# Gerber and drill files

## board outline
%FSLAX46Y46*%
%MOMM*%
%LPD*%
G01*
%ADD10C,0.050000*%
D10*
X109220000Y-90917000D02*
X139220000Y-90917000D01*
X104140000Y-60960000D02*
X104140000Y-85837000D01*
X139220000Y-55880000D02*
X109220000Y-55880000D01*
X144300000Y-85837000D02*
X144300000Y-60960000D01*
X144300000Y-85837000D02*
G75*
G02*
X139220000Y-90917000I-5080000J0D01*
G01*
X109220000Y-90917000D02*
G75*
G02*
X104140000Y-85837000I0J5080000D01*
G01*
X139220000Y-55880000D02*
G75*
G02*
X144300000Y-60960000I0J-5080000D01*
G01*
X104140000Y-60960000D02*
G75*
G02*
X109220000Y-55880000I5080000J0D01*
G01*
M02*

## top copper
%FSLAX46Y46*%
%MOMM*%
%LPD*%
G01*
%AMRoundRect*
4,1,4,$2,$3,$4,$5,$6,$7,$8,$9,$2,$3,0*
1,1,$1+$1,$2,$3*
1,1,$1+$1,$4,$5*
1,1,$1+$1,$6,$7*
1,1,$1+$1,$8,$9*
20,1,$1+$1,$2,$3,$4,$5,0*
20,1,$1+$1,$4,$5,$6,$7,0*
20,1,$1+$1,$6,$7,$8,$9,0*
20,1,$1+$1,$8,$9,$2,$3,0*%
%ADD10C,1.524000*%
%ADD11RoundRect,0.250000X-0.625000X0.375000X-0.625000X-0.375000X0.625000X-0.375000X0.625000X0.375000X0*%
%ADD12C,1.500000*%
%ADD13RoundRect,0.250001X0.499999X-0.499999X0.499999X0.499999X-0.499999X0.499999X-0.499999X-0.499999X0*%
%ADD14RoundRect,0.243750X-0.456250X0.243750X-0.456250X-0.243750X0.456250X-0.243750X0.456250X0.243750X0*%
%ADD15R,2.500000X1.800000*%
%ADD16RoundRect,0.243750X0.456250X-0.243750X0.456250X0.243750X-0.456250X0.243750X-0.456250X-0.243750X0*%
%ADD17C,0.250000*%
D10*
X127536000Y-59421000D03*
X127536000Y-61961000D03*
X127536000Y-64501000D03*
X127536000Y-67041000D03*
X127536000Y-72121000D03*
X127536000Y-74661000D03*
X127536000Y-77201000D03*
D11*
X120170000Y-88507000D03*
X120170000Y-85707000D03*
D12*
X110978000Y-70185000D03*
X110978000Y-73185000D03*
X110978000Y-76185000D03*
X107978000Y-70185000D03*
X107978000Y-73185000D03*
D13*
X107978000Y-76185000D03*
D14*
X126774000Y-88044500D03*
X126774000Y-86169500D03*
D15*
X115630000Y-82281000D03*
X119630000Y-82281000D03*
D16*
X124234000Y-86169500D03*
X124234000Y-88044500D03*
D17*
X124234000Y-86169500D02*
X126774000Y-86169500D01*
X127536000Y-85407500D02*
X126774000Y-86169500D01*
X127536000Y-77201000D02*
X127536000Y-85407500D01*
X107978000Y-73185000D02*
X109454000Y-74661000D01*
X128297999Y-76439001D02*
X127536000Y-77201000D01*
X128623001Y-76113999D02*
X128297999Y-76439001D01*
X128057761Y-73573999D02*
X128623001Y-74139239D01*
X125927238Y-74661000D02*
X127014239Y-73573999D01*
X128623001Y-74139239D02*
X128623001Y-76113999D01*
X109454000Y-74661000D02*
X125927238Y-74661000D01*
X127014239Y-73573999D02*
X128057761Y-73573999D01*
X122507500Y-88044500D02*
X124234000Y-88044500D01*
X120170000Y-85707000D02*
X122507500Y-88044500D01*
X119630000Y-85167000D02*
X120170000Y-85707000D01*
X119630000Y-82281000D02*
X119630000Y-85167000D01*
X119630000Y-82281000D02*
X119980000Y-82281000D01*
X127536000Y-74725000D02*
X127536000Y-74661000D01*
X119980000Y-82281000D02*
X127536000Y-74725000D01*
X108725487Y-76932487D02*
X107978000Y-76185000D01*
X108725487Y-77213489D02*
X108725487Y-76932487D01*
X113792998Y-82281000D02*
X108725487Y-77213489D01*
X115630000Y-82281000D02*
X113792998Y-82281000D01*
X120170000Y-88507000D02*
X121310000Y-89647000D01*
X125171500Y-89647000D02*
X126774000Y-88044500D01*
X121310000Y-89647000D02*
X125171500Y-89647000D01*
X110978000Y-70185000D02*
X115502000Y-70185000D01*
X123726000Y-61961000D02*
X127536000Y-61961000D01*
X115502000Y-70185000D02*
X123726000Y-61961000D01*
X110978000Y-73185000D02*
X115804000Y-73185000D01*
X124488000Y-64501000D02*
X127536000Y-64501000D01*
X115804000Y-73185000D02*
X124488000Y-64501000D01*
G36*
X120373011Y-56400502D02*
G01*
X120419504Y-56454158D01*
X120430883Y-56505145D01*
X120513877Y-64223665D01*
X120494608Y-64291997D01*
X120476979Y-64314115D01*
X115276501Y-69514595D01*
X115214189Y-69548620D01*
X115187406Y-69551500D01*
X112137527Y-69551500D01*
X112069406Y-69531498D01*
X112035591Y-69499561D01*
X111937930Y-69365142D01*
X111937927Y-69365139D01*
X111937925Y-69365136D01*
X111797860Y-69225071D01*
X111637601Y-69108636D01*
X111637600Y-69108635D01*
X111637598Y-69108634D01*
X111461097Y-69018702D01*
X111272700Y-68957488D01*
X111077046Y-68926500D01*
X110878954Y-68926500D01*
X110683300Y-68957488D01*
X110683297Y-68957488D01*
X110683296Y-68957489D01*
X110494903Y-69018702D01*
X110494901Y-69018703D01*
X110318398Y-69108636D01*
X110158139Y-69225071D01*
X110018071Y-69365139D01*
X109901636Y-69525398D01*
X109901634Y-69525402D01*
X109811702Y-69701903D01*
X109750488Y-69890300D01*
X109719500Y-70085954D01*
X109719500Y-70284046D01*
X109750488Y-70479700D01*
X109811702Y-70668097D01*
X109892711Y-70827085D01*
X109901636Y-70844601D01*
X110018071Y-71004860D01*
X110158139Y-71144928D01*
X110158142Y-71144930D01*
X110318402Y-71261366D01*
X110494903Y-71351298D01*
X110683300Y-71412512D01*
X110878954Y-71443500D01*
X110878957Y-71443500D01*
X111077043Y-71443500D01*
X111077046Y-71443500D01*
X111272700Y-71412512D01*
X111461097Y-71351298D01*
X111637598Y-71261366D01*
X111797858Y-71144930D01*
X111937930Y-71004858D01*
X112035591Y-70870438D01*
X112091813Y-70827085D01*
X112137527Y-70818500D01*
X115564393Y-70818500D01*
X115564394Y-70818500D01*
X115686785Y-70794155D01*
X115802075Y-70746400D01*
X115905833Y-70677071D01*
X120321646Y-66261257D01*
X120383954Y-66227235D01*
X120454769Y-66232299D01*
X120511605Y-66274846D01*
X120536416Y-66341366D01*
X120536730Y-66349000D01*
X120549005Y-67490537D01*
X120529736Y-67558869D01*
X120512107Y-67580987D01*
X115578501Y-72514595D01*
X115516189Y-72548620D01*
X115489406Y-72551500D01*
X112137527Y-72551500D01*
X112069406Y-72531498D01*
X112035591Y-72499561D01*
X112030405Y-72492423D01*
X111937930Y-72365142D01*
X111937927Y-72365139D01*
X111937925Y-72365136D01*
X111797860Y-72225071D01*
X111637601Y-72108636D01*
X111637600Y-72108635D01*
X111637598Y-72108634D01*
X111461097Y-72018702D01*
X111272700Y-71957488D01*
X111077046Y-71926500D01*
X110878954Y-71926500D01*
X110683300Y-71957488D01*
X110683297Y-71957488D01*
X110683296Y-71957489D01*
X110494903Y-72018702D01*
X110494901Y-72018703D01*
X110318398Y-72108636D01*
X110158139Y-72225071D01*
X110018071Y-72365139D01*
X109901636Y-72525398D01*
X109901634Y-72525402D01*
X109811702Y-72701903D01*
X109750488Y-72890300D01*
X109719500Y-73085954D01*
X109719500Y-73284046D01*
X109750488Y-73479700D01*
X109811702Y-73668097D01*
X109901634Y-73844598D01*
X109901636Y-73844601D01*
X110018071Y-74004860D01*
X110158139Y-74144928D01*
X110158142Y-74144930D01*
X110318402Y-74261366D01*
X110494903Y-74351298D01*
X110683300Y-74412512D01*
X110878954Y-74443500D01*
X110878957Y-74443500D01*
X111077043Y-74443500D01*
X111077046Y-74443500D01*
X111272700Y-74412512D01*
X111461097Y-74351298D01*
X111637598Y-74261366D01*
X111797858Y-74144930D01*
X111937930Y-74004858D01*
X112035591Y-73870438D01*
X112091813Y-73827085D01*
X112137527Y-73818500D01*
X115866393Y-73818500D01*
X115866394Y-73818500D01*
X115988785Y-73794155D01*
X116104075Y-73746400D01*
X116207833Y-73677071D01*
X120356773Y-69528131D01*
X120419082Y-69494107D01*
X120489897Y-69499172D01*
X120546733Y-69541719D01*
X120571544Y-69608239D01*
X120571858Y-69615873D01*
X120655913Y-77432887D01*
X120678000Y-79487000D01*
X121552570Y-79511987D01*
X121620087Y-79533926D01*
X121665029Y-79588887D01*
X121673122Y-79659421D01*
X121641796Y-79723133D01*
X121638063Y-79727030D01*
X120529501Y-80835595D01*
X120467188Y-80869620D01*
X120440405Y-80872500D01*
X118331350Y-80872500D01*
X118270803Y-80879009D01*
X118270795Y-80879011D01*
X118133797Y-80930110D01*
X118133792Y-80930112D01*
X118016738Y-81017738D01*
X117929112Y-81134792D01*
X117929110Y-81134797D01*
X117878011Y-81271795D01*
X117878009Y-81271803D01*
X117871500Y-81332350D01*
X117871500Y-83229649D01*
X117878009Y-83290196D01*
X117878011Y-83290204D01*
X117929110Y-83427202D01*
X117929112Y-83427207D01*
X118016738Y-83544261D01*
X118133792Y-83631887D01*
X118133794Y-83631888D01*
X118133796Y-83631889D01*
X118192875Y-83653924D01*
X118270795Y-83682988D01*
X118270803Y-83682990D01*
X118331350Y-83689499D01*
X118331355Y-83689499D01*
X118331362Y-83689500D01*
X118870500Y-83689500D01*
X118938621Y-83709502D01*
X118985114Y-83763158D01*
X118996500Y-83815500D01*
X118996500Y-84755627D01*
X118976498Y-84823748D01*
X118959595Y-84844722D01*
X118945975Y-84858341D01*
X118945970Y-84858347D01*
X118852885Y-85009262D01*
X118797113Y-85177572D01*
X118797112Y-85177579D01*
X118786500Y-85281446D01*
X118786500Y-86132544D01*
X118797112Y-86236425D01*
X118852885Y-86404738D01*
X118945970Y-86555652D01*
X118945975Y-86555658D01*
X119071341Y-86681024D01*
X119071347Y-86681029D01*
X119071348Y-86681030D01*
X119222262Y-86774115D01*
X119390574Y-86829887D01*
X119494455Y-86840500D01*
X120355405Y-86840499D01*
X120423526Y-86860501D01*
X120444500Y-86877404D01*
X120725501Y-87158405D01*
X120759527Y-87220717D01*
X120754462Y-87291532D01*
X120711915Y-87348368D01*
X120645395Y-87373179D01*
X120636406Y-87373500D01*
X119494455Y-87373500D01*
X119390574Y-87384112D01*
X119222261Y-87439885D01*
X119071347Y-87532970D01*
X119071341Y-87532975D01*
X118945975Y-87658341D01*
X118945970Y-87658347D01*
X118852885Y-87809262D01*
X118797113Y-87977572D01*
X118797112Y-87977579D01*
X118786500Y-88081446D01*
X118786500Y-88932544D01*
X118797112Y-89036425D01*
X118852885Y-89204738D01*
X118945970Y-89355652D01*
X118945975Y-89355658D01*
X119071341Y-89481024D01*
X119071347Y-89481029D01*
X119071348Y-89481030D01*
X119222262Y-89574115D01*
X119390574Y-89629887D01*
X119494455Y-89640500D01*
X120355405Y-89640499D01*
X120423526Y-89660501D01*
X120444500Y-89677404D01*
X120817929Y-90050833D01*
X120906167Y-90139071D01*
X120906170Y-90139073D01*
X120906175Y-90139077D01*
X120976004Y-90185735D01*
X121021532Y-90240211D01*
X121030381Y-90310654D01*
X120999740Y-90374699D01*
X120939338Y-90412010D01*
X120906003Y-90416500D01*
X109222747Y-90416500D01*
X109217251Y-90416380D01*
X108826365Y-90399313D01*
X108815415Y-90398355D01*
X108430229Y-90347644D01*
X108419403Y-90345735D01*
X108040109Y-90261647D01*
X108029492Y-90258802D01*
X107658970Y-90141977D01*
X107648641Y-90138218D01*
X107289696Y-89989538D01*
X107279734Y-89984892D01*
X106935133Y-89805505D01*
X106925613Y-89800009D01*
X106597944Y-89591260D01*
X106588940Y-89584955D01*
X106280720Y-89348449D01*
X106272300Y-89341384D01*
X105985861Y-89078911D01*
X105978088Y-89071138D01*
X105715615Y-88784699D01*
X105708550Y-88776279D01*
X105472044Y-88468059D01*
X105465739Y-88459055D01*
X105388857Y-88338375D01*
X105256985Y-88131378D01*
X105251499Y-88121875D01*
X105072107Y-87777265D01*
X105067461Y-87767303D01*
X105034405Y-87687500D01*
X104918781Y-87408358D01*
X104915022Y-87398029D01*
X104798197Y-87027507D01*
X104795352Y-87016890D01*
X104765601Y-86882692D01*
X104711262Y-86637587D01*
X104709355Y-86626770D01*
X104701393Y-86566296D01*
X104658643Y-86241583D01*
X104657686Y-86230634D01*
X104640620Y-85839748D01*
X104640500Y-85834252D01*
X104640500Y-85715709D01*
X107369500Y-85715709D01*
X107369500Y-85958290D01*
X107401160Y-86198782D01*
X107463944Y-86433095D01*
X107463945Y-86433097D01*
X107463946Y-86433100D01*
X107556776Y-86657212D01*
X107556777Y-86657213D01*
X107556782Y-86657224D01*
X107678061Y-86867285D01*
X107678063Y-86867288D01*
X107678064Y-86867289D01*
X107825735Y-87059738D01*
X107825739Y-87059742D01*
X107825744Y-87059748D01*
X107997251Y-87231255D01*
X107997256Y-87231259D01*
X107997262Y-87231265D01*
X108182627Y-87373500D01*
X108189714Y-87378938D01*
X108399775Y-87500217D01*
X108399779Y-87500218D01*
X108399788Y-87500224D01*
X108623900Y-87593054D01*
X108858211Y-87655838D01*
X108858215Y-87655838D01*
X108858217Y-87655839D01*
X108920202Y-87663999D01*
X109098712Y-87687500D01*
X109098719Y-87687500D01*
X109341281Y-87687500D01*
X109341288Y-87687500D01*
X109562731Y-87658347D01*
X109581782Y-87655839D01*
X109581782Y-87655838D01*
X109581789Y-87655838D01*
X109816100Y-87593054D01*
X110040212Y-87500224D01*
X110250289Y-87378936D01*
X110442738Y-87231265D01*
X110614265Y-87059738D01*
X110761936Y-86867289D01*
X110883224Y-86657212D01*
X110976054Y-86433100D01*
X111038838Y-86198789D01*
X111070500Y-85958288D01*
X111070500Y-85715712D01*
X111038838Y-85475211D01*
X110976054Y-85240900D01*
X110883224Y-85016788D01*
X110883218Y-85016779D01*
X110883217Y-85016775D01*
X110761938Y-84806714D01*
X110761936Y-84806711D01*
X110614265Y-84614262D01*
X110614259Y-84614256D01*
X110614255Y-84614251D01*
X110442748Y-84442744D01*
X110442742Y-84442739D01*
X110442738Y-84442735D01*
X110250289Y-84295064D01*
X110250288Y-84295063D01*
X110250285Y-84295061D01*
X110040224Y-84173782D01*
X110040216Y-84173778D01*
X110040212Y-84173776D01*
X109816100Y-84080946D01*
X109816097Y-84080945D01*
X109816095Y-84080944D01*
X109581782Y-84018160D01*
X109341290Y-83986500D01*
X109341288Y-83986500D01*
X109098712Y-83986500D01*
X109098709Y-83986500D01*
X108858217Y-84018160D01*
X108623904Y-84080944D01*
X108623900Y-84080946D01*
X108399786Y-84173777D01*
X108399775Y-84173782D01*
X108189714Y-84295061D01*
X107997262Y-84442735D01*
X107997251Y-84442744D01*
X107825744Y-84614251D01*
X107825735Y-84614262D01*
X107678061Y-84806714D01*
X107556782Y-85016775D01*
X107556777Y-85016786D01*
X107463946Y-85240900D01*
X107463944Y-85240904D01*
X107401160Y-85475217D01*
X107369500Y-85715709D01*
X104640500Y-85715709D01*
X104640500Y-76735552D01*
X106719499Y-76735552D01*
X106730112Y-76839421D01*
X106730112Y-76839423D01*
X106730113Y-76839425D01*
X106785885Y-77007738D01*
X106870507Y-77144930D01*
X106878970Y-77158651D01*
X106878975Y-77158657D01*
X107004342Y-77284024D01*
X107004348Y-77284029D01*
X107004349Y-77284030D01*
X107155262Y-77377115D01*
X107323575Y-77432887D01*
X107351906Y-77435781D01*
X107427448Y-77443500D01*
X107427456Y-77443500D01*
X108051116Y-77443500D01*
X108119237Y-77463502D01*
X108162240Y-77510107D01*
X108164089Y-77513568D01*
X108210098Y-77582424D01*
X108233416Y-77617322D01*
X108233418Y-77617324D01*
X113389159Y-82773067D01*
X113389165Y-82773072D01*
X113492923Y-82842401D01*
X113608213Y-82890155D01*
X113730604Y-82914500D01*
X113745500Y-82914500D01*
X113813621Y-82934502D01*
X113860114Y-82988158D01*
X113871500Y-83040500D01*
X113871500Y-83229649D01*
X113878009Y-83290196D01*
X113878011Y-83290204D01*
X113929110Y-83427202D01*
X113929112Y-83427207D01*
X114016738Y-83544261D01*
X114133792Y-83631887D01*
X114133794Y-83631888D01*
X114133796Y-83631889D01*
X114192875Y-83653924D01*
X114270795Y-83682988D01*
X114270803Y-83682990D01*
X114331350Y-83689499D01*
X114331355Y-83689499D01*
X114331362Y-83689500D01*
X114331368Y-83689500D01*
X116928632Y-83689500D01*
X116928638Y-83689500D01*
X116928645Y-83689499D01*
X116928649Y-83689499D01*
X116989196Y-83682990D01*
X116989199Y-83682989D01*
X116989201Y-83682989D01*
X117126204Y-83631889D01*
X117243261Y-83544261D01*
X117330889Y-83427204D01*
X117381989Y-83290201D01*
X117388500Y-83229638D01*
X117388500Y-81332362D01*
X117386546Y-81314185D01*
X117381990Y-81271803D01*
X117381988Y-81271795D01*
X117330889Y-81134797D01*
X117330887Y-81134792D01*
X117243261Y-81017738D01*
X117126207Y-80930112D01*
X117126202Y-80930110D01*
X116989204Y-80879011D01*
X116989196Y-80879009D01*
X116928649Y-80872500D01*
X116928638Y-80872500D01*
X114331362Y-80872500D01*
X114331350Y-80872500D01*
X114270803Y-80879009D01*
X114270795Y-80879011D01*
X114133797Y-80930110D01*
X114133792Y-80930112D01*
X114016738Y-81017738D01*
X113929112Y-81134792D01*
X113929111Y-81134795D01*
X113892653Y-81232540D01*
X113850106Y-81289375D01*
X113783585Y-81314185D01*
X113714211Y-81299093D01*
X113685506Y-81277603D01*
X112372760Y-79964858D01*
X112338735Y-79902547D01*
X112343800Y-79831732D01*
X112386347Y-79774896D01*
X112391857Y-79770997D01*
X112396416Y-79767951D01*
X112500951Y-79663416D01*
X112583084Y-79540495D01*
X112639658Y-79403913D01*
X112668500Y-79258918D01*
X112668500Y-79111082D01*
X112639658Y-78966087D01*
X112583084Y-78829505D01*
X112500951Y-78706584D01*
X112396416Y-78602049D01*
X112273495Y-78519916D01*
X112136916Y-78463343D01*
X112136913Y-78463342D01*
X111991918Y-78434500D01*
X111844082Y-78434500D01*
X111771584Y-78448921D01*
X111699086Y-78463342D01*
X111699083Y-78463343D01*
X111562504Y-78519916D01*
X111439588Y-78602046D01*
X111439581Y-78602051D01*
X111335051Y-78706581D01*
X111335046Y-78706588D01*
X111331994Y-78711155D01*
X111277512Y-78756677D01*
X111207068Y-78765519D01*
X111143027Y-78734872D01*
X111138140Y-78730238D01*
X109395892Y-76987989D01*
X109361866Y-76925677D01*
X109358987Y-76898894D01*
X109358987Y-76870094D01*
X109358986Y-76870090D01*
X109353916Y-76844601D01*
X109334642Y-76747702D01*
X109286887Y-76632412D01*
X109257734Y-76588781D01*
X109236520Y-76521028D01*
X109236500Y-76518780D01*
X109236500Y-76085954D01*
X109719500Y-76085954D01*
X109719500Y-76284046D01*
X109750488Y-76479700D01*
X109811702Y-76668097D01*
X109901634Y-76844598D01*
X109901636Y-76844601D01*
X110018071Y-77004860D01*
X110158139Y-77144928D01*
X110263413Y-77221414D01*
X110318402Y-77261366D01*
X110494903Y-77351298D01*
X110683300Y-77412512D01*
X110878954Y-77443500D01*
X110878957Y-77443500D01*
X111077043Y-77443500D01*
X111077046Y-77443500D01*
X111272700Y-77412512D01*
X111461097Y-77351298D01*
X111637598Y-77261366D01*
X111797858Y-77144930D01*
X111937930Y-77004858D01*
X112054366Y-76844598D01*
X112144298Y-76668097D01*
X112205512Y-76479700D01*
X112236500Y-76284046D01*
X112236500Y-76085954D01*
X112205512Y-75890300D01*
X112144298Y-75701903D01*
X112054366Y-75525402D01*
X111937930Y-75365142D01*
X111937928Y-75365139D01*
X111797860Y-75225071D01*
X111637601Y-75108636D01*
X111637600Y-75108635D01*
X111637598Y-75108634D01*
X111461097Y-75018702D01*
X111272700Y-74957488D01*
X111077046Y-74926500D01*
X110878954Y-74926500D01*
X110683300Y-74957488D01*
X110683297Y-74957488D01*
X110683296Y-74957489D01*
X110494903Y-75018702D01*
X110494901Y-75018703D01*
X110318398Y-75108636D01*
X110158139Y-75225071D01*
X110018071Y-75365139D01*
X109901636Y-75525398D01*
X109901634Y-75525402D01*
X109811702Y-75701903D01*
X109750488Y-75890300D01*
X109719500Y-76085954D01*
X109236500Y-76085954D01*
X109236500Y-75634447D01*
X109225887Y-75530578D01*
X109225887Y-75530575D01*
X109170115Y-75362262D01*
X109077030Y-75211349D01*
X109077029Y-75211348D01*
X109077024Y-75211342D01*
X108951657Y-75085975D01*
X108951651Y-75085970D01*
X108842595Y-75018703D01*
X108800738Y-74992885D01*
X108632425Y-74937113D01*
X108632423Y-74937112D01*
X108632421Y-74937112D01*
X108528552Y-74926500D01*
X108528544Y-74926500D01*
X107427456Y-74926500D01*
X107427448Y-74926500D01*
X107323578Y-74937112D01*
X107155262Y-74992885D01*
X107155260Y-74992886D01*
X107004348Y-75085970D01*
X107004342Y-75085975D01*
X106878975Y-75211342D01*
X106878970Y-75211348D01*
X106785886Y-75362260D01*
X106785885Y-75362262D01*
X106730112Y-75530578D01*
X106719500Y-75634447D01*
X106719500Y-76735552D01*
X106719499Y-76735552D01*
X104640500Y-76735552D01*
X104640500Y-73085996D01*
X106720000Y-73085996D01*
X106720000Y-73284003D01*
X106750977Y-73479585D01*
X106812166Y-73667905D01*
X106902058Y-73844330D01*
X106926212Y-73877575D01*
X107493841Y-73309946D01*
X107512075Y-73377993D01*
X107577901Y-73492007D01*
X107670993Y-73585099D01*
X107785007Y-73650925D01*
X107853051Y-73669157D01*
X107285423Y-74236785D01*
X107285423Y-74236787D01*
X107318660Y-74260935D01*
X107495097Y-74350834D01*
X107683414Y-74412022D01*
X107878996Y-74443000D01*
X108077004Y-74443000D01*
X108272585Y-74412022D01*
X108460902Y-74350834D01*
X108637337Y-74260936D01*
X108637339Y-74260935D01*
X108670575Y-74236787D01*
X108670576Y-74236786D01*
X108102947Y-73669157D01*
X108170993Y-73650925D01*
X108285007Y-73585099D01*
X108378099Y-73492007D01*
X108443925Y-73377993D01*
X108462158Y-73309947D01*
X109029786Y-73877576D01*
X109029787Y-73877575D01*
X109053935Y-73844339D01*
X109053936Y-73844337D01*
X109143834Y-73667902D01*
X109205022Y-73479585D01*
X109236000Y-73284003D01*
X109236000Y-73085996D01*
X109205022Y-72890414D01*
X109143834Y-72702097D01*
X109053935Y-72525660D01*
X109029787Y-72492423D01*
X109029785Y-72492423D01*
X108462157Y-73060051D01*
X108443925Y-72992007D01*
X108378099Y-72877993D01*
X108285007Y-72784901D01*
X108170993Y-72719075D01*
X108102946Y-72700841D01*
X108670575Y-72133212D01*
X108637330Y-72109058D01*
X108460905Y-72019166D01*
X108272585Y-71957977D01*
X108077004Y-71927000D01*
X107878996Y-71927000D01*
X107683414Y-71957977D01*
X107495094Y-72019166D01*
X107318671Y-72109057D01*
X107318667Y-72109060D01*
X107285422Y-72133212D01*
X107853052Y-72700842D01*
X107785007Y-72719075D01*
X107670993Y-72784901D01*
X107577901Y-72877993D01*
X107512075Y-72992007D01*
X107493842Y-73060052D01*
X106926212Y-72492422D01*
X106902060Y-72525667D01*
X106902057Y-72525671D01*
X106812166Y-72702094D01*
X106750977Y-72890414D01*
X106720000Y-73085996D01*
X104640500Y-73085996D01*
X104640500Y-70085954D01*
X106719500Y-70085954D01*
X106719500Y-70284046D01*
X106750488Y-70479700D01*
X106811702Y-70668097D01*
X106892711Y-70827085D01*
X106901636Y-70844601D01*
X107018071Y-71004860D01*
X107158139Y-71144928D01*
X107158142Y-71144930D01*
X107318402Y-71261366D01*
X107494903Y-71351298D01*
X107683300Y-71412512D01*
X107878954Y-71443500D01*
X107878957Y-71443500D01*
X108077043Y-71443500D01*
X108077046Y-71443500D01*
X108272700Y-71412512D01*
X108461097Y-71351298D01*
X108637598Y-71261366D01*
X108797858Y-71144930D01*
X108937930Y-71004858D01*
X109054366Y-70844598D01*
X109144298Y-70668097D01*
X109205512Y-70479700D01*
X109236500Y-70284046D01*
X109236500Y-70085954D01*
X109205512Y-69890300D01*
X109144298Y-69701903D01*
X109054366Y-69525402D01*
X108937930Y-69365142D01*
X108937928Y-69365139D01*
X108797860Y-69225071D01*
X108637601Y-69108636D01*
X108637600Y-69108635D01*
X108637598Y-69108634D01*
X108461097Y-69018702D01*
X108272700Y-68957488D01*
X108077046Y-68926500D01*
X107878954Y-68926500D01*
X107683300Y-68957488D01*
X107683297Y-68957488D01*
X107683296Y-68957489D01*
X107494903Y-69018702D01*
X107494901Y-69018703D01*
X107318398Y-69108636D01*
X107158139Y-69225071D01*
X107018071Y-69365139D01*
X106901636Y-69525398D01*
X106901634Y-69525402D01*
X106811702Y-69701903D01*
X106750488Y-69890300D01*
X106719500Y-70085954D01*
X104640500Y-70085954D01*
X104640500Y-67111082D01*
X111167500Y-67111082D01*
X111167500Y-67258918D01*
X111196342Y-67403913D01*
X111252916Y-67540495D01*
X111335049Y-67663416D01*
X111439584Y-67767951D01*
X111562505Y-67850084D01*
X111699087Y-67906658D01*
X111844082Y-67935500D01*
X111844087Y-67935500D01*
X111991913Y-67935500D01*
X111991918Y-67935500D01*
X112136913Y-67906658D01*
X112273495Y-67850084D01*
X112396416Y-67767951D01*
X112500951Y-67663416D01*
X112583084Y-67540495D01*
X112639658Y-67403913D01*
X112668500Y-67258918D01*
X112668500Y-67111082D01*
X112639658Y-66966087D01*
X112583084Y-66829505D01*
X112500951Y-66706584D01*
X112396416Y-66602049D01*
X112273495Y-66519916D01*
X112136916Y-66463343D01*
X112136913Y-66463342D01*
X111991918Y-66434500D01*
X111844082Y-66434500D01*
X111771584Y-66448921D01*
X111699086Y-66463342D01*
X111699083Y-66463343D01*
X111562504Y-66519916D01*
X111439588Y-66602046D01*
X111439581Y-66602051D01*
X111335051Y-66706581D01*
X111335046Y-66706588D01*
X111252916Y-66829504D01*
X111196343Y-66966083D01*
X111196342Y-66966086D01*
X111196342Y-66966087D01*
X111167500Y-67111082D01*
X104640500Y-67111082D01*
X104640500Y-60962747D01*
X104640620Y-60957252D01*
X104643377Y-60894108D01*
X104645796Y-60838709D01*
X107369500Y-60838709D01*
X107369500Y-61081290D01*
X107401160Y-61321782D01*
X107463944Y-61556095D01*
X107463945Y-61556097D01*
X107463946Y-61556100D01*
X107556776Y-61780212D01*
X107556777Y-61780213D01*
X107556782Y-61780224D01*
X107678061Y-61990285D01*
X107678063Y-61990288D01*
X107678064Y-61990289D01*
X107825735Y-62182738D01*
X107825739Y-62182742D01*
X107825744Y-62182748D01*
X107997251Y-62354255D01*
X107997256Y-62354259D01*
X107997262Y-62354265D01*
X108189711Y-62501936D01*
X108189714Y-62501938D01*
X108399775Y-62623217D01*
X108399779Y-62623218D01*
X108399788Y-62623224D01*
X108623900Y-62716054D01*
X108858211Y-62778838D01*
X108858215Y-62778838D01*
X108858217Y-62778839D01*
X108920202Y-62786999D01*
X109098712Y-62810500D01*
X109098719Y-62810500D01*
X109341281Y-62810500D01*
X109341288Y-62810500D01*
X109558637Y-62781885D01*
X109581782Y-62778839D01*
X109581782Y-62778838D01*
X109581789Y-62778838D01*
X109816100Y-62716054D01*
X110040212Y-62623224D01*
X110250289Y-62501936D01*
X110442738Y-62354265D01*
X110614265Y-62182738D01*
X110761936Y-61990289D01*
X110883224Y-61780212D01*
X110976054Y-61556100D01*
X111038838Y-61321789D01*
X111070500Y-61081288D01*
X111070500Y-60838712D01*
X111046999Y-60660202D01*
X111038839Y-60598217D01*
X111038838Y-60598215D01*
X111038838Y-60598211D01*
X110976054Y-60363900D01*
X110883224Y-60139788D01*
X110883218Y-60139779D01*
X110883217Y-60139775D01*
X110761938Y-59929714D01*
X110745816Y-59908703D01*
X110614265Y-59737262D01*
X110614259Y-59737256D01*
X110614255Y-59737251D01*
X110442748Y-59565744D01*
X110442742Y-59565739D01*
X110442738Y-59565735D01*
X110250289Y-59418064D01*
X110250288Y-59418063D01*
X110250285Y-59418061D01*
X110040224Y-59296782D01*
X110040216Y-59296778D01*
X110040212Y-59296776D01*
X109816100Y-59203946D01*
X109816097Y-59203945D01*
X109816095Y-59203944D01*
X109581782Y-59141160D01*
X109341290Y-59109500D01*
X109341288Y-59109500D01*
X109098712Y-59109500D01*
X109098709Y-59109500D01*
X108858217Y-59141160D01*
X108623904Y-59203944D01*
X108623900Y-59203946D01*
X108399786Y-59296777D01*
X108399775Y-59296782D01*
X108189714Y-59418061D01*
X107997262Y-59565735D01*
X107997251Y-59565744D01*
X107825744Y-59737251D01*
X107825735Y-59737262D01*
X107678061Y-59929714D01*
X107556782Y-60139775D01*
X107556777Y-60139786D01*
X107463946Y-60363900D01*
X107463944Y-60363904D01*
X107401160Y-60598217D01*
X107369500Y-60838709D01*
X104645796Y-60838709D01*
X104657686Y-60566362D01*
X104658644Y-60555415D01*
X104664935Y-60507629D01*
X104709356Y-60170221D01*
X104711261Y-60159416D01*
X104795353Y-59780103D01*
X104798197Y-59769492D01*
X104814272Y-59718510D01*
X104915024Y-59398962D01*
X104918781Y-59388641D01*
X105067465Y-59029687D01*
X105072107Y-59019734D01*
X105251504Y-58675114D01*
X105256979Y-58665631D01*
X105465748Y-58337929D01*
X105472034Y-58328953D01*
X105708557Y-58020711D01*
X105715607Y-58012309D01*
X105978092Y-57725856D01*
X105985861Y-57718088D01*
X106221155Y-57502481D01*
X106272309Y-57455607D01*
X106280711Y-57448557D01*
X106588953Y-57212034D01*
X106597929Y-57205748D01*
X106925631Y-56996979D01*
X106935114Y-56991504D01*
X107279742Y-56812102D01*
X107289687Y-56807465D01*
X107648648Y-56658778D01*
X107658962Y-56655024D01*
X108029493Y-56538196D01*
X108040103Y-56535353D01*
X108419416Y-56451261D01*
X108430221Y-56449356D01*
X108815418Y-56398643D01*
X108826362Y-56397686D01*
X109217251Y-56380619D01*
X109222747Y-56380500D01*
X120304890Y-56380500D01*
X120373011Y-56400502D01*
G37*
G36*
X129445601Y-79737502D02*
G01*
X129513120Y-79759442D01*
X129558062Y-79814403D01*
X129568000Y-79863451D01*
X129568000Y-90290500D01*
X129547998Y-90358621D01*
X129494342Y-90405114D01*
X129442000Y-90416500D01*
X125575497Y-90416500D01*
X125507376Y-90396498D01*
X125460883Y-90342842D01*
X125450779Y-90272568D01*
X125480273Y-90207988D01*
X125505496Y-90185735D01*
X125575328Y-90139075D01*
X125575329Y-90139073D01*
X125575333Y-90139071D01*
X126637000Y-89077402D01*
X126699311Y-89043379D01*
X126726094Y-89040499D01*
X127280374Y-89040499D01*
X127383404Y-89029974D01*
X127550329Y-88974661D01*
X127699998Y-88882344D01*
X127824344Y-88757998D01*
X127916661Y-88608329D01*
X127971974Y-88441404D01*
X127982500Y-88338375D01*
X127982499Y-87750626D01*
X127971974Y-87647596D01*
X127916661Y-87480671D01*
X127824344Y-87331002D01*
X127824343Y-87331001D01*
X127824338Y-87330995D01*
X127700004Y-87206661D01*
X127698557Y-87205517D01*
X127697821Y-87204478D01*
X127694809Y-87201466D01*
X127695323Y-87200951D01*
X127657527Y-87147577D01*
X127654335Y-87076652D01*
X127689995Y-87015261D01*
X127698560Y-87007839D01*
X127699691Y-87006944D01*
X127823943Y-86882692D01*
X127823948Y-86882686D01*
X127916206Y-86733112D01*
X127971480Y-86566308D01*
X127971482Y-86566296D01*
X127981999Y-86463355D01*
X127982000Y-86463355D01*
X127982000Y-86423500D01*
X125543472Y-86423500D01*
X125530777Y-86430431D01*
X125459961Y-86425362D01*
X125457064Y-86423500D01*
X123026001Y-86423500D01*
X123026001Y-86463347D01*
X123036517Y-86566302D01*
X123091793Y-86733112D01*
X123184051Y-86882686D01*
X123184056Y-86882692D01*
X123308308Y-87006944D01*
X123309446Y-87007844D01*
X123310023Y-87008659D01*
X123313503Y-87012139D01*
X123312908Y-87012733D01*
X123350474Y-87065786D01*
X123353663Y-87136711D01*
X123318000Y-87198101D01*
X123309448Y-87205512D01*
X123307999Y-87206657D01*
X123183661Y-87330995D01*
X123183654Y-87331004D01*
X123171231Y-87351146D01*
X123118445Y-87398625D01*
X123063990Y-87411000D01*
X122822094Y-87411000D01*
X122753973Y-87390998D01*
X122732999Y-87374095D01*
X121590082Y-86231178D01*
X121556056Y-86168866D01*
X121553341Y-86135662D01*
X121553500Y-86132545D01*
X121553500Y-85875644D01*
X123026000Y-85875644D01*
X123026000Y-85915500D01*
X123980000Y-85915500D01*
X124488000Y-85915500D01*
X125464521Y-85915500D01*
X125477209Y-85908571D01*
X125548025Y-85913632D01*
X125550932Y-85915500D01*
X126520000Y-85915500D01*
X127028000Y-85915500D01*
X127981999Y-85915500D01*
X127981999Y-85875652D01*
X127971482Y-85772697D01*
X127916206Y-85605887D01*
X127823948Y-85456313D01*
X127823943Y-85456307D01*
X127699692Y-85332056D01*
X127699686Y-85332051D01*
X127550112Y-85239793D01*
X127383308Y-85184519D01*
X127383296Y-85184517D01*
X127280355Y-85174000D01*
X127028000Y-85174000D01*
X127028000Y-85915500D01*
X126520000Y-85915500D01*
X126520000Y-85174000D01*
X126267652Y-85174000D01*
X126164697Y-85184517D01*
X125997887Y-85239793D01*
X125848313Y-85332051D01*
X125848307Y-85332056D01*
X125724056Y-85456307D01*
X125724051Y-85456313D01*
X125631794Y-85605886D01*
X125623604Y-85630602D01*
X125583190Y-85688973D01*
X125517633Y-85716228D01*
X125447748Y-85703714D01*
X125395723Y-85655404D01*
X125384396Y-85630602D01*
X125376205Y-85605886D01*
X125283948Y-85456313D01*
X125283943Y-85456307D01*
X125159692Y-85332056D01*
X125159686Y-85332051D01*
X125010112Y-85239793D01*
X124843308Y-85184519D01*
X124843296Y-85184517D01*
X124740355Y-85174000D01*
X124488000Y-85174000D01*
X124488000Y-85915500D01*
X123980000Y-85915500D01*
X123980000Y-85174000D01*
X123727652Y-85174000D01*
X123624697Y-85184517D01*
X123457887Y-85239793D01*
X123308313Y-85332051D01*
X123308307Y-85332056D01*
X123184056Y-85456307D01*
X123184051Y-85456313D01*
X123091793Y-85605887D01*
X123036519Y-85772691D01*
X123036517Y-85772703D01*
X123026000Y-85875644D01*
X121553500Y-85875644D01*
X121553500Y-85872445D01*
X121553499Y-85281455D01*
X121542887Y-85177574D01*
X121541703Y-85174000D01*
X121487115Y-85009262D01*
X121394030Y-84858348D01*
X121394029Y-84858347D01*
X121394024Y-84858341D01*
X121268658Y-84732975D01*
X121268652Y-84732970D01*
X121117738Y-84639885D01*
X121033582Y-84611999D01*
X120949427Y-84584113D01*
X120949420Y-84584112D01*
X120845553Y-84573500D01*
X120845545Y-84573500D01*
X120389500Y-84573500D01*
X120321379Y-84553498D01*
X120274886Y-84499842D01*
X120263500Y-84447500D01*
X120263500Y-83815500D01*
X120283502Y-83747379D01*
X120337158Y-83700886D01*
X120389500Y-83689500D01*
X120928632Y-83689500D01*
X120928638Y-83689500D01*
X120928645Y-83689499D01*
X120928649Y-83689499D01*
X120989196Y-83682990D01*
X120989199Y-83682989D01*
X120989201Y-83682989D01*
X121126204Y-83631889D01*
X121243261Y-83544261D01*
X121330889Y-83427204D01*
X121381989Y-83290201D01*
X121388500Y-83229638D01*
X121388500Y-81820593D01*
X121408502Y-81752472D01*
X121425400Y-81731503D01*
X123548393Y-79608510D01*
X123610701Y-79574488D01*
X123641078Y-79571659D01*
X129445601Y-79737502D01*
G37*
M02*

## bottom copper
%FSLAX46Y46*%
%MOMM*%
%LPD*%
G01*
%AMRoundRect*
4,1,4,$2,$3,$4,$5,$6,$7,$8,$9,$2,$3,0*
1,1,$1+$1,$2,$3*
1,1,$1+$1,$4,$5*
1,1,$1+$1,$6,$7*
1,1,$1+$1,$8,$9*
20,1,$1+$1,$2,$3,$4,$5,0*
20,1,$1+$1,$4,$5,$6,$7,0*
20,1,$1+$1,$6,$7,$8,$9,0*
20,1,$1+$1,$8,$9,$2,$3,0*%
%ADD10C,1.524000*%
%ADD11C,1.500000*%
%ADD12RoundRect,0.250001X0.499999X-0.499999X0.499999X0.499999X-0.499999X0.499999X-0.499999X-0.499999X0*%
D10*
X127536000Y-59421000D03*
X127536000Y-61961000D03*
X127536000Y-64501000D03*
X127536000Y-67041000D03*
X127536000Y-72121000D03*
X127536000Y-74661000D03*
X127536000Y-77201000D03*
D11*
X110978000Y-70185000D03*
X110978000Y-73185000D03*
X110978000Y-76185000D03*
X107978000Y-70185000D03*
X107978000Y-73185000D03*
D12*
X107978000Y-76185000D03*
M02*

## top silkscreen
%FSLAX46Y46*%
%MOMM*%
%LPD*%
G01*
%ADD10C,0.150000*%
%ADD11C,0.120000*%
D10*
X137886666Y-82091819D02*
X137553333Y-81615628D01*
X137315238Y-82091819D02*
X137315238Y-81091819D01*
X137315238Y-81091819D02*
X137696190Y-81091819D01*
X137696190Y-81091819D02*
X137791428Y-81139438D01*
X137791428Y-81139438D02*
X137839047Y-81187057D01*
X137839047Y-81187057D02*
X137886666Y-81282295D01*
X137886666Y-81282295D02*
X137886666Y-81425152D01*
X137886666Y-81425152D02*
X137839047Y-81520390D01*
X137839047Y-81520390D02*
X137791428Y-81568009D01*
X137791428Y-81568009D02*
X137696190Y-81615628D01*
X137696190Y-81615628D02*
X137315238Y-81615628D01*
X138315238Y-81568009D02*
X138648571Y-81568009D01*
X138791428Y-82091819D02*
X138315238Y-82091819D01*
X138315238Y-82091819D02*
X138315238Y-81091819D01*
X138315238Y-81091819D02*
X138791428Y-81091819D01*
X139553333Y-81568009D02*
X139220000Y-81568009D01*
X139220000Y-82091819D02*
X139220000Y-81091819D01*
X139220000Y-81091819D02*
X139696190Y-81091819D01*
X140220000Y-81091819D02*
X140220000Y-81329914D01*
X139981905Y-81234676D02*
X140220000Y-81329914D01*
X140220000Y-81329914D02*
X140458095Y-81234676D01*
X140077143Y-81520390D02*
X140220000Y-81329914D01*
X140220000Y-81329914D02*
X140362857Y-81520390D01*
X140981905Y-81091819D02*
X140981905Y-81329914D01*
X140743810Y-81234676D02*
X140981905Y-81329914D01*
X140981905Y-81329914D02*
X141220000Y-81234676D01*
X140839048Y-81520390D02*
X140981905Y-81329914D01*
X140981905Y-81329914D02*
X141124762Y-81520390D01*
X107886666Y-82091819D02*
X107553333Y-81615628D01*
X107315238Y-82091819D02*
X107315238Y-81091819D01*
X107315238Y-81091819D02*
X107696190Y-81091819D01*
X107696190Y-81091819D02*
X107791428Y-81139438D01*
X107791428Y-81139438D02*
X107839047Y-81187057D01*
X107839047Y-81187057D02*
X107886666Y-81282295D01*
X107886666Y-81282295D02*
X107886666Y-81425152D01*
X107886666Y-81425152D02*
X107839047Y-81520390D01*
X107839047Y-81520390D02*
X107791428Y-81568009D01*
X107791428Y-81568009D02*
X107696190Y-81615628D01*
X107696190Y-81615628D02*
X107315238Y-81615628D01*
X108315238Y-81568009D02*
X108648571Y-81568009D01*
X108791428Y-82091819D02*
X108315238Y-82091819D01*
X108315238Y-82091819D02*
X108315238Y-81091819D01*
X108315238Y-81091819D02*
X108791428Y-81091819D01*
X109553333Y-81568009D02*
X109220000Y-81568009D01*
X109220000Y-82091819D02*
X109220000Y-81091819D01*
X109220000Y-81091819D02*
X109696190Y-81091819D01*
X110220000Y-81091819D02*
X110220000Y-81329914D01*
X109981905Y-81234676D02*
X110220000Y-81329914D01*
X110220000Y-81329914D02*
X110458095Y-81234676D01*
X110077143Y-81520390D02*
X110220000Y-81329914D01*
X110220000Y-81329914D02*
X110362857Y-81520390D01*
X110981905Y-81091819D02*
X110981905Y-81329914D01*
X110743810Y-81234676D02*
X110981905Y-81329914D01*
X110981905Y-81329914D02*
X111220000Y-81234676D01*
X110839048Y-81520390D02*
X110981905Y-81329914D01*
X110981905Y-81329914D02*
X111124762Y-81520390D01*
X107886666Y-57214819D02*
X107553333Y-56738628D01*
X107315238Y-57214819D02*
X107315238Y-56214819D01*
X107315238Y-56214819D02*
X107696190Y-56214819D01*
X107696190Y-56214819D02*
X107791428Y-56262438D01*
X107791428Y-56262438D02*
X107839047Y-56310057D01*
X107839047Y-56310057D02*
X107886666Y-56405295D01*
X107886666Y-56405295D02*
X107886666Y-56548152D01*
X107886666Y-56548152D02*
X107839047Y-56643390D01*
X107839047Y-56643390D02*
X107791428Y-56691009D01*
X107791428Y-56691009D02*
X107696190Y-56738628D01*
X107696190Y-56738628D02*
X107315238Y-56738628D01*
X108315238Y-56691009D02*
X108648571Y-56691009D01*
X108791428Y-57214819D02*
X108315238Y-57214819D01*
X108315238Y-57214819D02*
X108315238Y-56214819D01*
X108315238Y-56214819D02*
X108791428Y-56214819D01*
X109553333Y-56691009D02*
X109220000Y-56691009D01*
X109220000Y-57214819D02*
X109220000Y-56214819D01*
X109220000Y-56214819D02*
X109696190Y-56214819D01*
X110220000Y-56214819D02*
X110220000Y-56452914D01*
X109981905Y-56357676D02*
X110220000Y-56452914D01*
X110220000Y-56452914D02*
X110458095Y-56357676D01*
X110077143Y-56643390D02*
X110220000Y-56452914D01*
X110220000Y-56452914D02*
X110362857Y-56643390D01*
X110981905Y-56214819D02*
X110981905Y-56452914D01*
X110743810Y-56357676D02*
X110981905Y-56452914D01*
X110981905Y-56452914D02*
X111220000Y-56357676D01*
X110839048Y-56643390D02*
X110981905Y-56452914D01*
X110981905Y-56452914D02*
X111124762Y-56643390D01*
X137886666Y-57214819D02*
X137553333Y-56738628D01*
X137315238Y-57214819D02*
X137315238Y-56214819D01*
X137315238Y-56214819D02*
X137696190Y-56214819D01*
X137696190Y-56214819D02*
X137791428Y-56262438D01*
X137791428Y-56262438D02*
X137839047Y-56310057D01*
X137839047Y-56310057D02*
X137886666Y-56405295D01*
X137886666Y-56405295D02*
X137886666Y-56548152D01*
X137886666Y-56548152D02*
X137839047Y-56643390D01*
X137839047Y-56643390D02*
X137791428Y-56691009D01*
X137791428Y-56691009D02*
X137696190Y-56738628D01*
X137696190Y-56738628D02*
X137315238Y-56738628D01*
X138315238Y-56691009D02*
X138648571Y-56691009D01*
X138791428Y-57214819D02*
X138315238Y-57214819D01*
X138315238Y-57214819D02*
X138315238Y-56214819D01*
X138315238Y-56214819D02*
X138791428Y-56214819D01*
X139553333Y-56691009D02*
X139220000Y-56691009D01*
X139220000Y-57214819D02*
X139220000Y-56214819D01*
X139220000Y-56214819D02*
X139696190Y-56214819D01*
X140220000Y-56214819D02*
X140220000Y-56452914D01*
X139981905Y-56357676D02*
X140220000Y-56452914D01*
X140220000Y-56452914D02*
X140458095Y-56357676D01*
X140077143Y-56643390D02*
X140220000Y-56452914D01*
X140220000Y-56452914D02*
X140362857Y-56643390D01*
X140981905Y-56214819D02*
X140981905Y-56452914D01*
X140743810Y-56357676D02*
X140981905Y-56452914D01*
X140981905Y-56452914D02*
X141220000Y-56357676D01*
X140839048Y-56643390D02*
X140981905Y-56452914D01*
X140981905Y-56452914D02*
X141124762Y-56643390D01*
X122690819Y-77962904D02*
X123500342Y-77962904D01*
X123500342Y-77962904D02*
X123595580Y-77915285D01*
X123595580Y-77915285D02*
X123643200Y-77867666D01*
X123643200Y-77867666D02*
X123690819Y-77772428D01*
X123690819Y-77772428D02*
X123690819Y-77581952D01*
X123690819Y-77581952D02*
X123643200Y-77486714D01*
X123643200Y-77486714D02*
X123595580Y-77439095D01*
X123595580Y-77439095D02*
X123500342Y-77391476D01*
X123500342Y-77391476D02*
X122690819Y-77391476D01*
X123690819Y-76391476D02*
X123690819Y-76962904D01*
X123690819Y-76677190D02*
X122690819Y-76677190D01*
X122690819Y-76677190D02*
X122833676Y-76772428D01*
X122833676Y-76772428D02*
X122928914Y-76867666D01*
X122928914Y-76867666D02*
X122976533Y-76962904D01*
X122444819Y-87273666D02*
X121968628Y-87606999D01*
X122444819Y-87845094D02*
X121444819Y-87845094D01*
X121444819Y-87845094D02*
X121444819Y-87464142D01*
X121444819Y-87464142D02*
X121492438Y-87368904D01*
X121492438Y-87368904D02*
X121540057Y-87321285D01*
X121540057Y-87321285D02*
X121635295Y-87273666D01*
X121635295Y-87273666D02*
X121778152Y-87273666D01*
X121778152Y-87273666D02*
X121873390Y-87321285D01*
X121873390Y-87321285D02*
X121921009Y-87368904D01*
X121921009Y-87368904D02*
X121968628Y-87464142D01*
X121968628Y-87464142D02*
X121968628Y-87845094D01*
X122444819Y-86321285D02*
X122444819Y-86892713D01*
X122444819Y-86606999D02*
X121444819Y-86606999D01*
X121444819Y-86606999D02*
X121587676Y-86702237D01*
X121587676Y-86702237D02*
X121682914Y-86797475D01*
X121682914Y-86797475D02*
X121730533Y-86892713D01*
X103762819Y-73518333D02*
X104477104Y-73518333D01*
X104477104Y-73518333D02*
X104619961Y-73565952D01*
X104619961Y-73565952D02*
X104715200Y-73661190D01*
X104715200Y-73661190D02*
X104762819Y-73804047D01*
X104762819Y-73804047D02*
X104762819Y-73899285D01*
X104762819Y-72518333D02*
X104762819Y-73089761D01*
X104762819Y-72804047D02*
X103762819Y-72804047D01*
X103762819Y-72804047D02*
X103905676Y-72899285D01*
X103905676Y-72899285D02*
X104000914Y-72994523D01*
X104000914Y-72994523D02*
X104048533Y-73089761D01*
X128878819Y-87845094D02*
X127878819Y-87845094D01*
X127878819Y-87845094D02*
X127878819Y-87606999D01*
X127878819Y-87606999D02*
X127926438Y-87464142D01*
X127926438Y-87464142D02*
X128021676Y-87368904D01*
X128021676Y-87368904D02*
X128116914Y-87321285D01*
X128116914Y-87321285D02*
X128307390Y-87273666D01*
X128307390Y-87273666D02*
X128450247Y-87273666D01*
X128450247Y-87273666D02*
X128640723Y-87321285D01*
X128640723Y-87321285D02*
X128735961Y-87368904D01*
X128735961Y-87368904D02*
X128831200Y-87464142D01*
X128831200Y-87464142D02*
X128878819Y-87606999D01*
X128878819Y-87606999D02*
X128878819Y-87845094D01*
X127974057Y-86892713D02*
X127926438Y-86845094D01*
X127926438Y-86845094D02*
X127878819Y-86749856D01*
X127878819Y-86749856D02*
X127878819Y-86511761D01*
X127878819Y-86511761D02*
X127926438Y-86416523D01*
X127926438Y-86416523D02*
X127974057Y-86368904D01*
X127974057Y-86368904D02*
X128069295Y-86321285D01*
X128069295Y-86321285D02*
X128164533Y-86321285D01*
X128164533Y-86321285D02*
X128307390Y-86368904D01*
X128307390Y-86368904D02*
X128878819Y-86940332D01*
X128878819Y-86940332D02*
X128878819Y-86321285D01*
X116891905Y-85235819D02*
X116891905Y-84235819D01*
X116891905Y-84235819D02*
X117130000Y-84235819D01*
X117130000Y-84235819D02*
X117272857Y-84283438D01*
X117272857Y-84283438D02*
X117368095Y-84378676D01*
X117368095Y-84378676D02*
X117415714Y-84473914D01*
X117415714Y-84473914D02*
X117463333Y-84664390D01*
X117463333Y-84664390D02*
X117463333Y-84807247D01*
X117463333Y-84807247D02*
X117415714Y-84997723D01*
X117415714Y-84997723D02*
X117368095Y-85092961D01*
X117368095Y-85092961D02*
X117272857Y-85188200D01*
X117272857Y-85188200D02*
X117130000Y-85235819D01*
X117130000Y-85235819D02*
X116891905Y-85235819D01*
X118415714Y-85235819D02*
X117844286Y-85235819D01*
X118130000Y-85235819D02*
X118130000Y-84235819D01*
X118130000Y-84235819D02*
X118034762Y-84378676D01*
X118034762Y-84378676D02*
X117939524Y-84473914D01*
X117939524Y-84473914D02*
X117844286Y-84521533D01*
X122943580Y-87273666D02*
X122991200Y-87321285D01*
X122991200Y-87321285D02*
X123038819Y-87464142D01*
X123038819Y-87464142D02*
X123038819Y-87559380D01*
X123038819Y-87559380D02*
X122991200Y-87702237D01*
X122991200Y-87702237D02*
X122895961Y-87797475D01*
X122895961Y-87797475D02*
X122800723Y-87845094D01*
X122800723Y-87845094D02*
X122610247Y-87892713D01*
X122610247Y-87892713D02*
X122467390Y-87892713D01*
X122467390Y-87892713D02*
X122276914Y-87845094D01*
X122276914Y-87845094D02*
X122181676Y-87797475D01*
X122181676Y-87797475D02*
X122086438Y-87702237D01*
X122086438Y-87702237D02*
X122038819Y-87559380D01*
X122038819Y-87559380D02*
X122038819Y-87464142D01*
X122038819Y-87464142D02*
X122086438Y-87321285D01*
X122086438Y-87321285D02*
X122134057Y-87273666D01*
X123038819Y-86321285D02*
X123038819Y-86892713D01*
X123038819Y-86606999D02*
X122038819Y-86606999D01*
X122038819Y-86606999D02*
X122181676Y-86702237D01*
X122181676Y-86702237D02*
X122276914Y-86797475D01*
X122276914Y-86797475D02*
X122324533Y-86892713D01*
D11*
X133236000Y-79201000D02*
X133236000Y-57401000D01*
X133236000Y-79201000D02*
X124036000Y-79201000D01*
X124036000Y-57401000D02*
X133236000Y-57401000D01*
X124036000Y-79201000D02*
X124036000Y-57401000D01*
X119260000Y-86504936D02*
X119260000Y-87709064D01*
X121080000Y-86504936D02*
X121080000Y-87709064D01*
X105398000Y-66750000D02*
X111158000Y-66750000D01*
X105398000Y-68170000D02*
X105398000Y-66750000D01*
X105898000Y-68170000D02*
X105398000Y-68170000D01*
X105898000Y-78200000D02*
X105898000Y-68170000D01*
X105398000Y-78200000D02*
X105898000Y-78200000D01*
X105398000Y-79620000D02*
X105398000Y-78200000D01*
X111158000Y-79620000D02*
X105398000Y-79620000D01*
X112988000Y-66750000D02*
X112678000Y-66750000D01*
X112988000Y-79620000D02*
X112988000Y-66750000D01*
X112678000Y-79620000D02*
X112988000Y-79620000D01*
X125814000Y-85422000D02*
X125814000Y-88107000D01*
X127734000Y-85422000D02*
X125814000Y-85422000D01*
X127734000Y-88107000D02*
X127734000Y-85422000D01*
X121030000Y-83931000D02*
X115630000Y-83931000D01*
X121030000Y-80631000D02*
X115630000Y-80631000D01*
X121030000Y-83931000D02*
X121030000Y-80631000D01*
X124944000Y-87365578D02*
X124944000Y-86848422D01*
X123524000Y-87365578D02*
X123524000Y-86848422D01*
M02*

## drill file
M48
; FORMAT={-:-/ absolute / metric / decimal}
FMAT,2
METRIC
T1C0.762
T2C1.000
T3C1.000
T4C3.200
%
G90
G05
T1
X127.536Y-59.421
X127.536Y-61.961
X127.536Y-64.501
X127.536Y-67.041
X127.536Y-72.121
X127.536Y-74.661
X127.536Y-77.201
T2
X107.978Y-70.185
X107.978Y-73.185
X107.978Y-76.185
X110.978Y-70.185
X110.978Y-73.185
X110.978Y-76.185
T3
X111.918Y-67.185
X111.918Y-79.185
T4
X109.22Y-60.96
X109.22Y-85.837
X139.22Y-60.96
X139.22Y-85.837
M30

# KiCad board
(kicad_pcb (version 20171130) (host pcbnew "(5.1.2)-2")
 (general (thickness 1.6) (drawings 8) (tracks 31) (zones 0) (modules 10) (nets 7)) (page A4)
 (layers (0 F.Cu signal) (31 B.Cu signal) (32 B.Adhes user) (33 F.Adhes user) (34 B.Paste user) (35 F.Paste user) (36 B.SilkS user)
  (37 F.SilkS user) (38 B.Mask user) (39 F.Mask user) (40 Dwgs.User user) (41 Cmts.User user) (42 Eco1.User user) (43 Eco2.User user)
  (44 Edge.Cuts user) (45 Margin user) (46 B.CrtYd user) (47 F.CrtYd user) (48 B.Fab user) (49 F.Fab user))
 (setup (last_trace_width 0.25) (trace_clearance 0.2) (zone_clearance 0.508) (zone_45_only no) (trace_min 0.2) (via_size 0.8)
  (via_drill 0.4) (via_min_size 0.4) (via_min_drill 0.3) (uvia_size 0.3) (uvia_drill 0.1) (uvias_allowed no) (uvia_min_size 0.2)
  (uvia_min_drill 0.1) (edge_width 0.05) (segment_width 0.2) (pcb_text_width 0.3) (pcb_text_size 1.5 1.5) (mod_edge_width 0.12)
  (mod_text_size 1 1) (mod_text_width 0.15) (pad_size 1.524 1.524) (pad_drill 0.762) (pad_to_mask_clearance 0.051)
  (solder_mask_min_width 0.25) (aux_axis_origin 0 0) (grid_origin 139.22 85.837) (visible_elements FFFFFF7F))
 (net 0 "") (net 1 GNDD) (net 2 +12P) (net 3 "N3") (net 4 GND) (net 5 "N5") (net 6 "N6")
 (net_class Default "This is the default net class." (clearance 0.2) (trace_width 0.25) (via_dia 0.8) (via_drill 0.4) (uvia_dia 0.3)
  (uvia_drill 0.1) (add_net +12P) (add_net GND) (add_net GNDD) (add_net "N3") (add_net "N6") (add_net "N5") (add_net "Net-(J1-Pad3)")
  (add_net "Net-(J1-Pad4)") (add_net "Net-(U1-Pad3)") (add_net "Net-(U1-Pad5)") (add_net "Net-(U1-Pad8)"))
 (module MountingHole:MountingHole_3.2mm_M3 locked (layer F.Cu) (at 139.22 85.837)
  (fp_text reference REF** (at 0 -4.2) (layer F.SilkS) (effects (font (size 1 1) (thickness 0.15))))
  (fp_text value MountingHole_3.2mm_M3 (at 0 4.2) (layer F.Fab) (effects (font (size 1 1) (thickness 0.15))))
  (pad 1 np_thru_hole circle (at 0 0) (size 3.2 3.2) (drill 3.2) (layers *.Cu *.Mask)))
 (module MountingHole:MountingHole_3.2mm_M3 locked (layer F.Cu) (at 109.22 85.837)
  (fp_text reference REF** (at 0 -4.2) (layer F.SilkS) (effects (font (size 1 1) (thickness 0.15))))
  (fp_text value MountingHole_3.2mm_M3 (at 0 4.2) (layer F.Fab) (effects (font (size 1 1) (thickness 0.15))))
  (pad 1 np_thru_hole circle (at 0 0) (size 3.2 3.2) (drill 3.2) (layers *.Cu *.Mask)))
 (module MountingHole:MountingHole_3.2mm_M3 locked (layer F.Cu) (at 109.22 60.96)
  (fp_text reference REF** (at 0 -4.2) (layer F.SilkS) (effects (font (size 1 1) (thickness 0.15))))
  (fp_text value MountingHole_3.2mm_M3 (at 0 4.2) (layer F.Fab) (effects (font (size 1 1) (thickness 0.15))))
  (pad 1 np_thru_hole circle (at 0 0) (size 3.2 3.2) (drill 3.2) (layers *.Cu *.Mask)))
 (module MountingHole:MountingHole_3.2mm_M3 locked (layer F.Cu) (at 139.22 60.96)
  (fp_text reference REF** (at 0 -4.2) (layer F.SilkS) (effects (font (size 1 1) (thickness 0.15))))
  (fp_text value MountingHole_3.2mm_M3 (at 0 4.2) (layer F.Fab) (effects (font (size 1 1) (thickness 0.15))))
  (pad 1 np_thru_hole circle (at 0 0) (size 3.2 3.2) (drill 3.2) (layers *.Cu *.Mask)))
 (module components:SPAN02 (layer F.Cu) (at 127.536 77.201 90)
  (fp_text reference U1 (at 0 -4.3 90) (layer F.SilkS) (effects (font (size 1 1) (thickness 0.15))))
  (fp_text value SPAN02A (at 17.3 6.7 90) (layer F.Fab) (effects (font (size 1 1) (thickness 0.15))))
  (fp_line (start -2 5.7) (end 19.8 5.7) (layer F.SilkS) (width 0.12))
  (fp_line (start -2 5.7) (end -2 -3.5) (layer F.SilkS) (width 0.12))
  (fp_line (start 19.8 -3.5) (end 19.8 5.7) (layer F.SilkS) (width 0.12))
  (fp_line (start -2 -3.5) (end 19.8 -3.5) (layer F.SilkS) (width 0.12))
  (pad 8 thru_hole circle (at 17.78 0 90) (size 1.524 1.524) (drill 0.762) (layers *.Cu *.Mask))
  (pad 7 thru_hole circle (at 15.24 0 90) (size 1.524 1.524) (drill 0.762) (layers *.Cu *.Mask) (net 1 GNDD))
  (pad 6 thru_hole circle (at 12.7 0 90) (size 1.524 1.524) (drill 0.762) (layers *.Cu *.Mask) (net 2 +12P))
  (pad 5 thru_hole circle (at 10.16 0 90) (size 1.524 1.524) (drill 0.762) (layers *.Cu *.Mask))
  (pad 3 thru_hole circle (at 5.08 0 90) (size 1.524 1.524) (drill 0.762) (layers *.Cu *.Mask))
  (pad 2 thru_hole circle (at 2.54 0 90) (size 1.524 1.524) (drill 0.762) (layers *.Cu *.Mask) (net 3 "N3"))
  (pad 1 thru_hole circle (at 0 0 90) (size 1.524 1.524) (drill 0.762) (layers *.Cu *.Mask) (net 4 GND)))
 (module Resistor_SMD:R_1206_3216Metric (layer F.Cu) (at 120.17 87.107 270)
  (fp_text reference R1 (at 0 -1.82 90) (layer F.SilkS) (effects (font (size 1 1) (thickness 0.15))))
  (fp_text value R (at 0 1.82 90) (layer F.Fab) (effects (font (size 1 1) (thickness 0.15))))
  (fp_line (start -0.602064 0.91) (end 0.602064 0.91) (layer F.SilkS) (width 0.12))
  (fp_line (start -0.602064 -0.91) (end 0.602064 -0.91) (layer F.SilkS) (width 0.12))
  (pad 2 smd roundrect (at 1.4 0 270) (size 1.25 1.75) (layers F.Cu F.Paste F.Mask) (roundrect_rratio 0.2) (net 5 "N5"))
  (pad 1 smd roundrect (at -1.4 0 270) (size 1.25 1.75) (layers F.Cu F.Paste F.Mask) (roundrect_rratio 0.2) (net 3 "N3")))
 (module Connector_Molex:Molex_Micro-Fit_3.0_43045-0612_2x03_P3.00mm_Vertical (layer F.Cu) (at 107.978 76.185 90)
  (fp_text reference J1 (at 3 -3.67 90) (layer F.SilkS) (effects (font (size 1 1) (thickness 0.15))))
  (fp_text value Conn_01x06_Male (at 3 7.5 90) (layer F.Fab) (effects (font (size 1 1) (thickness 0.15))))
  (fp_line (start 9.435 -2.58) (end 9.435 3.18) (layer F.SilkS) (width 0.12))
  (fp_line (start 8.015 -2.58) (end 9.435 -2.58) (layer F.SilkS) (width 0.12))
  (fp_line (start 8.015 -2.08) (end 8.015 -2.58) (layer F.SilkS) (width 0.12))
  (fp_line (start -2.015 -2.08) (end 8.015 -2.08) (layer F.SilkS) (width 0.12))
  (fp_line (start -2.015 -2.58) (end -2.015 -2.08) (layer F.SilkS) (width 0.12))
  (fp_line (start -3.435 -2.58) (end -2.015 -2.58) (layer F.SilkS) (width 0.12))
  (fp_line (start -3.435 3.18) (end -3.435 -2.58) (layer F.SilkS) (width 0.12))
  (fp_line (start 9.435 5.01) (end 9.435 4.7) (layer F.SilkS) (width 0.12))
  (fp_line (start -3.435 5.01) (end 9.435 5.01) (layer F.SilkS) (width 0.12))
  (fp_line (start -3.435 4.7) (end -3.435 5.01) (layer F.SilkS) (width 0.12))
  (pad 6 thru_hole circle (at 6 3 90) (size 1.5 1.5) (drill 1) (layers *.Cu *.Mask) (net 1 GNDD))
  (pad 5 thru_hole circle (at 3 3 90) (size 1.5 1.5) (drill 1) (layers *.Cu *.Mask) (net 2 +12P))
  (pad 4 thru_hole circle (at 0 3 90) (size 1.5 1.5) (drill 1) (layers *.Cu *.Mask))
  (pad 3 thru_hole circle (at 6 0 90) (size 1.5 1.5) (drill 1) (layers *.Cu *.Mask))
  (pad 2 thru_hole circle (at 3 0 90) (size 1.5 1.5) (drill 1) (layers *.Cu *.Mask) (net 4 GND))
  (pad 1 thru_hole roundrect (at 0 0 90) (size 1.5 1.5) (drill 1) (layers *.Cu *.Mask) (roundrect_rratio 0.166667) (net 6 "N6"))
  (pad "" np_thru_hole circle (at 9 3.94 90) (size 1 1) (drill 1) (layers *.Cu *.Mask))
  (pad "" np_thru_hole circle (at -3 3.94 90) (size 1 1) (drill 1) (layers *.Cu *.Mask)))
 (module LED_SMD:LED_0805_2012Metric (layer F.Cu) (at 126.774 87.107 270)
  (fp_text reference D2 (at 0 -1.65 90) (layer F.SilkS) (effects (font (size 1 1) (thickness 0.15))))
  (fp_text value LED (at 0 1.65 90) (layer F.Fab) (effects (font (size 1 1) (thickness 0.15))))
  (fp_line (start -1.685 0.96) (end 1 0.96) (layer F.SilkS) (width 0.12))
  (fp_line (start -1.685 -0.96) (end -1.685 0.96) (layer F.SilkS) (width 0.12))
  (fp_line (start 1 -0.96) (end -1.685 -0.96) (layer F.SilkS) (width 0.12))
  (pad 2 smd roundrect (at 0.9375 0 270) (size 0.975 1.4) (layers F.Cu F.Paste F.Mask) (roundrect_rratio 0.25) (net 5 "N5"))
  (pad 1 smd roundrect (at -0.9375 0 270) (size 0.975 1.4) (layers F.Cu F.Paste F.Mask) (roundrect_rratio 0.25) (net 4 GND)))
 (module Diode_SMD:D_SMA (layer F.Cu) (at 117.63 82.281 180)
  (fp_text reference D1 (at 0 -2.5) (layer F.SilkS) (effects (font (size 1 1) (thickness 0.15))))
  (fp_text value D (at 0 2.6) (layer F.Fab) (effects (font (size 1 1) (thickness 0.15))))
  (fp_line (start -3.4 -1.65) (end 2 -1.65) (layer F.SilkS) (width 0.12))
  (fp_line (start -3.4 1.65) (end 2 1.65) (layer F.SilkS) (width 0.12))
  (fp_line (start -3.4 -1.65) (end -3.4 1.65) (layer F.SilkS) (width 0.12))
  (pad 2 smd rect (at 2 0 180) (size 2.5 1.8) (layers F.Cu F.Paste F.Mask) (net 6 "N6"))
  (pad 1 smd rect (at -2 0 180) (size 2.5 1.8) (layers F.Cu F.Paste F.Mask) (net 3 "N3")))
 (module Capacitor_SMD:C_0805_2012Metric (layer F.Cu) (at 124.234 87.107 90)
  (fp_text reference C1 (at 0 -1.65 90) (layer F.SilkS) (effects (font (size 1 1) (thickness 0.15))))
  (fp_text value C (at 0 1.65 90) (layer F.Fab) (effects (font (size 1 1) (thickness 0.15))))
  (fp_line (start -0.258578 0.71) (end 0.258578 0.71) (layer F.SilkS) (width 0.12))
  (fp_line (start -0.258578 -0.71) (end 0.258578 -0.71) (layer F.SilkS) (width 0.12))
  (pad 2 smd roundrect (at 0.9375 0 90) (size 0.975 1.4) (layers F.Cu F.Paste F.Mask) (roundrect_rratio 0.25) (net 4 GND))
  (pad 1 smd roundrect (at -0.9375 0 90) (size 0.975 1.4) (layers F.Cu F.Paste F.Mask) (roundrect_rratio 0.25) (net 3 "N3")))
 (gr_line (start 109.22 90.917) (end 139.22 90.917) (layer Edge.Cuts) (width 0.05))
 (gr_line (start 104.14 60.96) (end 104.14 85.837) (layer Edge.Cuts) (width 0.05))
 (gr_line (start 139.22 55.88) (end 109.22 55.88) (layer Edge.Cuts) (width 0.05))
 (gr_line (start 144.3 85.837) (end 144.3 60.96) (layer Edge.Cuts) (width 0.05))
 (gr_arc (start 139.22 85.837) (end 139.22 90.917) (angle -90) (layer Edge.Cuts) (width 0.05))
 (gr_arc (start 109.22 85.837) (end 104.14 85.837) (angle -90) (layer Edge.Cuts) (width 0.05))
 (gr_arc (start 139.22 60.96) (end 144.3 60.96) (angle -90) (layer Edge.Cuts) (width 0.05))
 (gr_arc (start 109.22 60.96) (end 109.22 55.88) (angle -90) (layer Edge.Cuts) (width 0.05))
 (segment (start 124.234 86.1695) (end 126.774 86.1695) (width 0.25) (layer F.Cu) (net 4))
 (segment (start 127.536 85.4075) (end 126.774 86.1695) (width 0.25) (layer F.Cu) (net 4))
 (segment (start 127.536 77.201) (end 127.536 85.4075) (width 0.25) (layer F.Cu) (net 4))
 (segment (start 107.978 73.185) (end 109.454 74.661) (width 0.25) (layer F.Cu) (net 4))
 (segment (start 128.297999 76.439001) (end 127.536 77.201) (width 0.25) (layer F.Cu) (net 4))
 (segment (start 128.623001 76.113999) (end 128.297999 76.439001) (width 0.25) (layer F.Cu) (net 4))
 (segment (start 128.057761 73.573999) (end 128.623001 74.139239) (width 0.25) (layer F.Cu) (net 4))
 (segment (start 125.927238 74.661) (end 127.014239 73.573999) (width 0.25) (layer F.Cu) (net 4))
 (segment (start 128.623001 74.139239) (end 128.623001 76.113999) (width 0.25) (layer F.Cu) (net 4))
 (segment (start 109.454 74.661) (end 125.927238 74.661) (width 0.25) (layer F.Cu) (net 4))
 (segment (start 127.014239 73.573999) (end 128.057761 73.573999) (width 0.25) (layer F.Cu) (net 4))
 (segment (start 122.5075 88.0445) (end 124.234 88.0445) (width 0.25) (layer F.Cu) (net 3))
 (segment (start 120.17 85.707) (end 122.5075 88.0445) (width 0.25) (layer F.Cu) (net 3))
 (segment (start 119.63 85.167) (end 120.17 85.707) (width 0.25) (layer F.Cu) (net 3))
 (segment (start 119.63 82.281) (end 119.63 85.167) (width 0.25) (layer F.Cu) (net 3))
 (segment (start 119.63 82.281) (end 119.98 82.281) (width 0.25) (layer F.Cu) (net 3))
 (segment (start 127.536 74.725) (end 127.536 74.661) (width 0.25) (layer F.Cu) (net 3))
 (segment (start 119.98 82.281) (end 127.536 74.725) (width 0.25) (layer F.Cu) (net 3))
 (segment (start 108.725487 76.932487) (end 107.978 76.185) (width 0.25) (layer F.Cu) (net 6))
 (segment (start 108.725487 77.213489) (end 108.725487 76.932487) (width 0.25) (layer F.Cu) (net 6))
 (segment (start 113.792998 82.281) (end 108.725487 77.213489) (width 0.25) (layer F.Cu) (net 6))
 (segment (start 115.63 82.281) (end 113.792998 82.281) (width 0.25) (layer F.Cu) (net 6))
 (segment (start 120.17 88.507) (end 121.31 89.647) (width 0.25) (layer F.Cu) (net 5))
 (segment (start 125.1715 89.647) (end 126.774 88.0445) (width 0.25) (layer F.Cu) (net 5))
 (segment (start 121.31 89.647) (end 125.1715 89.647) (width 0.25) (layer F.Cu) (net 5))
 (segment (start 110.978 70.185) (end 115.502 70.185) (width 0.25) (layer F.Cu) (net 1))
 (segment (start 123.726 61.961) (end 127.536 61.961) (width 0.25) (layer F.Cu) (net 1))
 (segment (start 115.502 70.185) (end 123.726 61.961) (width 0.25) (layer F.Cu) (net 1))
 (segment (start 110.978 73.185) (end 115.804 73.185) (width 0.25) (layer F.Cu) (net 2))
 (segment (start 124.488 64.501) (end 127.536 64.501) (width 0.25) (layer F.Cu) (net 2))
 (segment (start 115.804 73.185) (end 124.488 64.501) (width 0.25) (layer F.Cu) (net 2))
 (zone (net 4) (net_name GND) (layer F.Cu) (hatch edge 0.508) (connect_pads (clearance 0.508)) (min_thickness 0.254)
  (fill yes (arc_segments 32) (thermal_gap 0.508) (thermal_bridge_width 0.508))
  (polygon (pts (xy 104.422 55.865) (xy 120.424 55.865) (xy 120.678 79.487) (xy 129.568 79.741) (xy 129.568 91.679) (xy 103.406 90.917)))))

